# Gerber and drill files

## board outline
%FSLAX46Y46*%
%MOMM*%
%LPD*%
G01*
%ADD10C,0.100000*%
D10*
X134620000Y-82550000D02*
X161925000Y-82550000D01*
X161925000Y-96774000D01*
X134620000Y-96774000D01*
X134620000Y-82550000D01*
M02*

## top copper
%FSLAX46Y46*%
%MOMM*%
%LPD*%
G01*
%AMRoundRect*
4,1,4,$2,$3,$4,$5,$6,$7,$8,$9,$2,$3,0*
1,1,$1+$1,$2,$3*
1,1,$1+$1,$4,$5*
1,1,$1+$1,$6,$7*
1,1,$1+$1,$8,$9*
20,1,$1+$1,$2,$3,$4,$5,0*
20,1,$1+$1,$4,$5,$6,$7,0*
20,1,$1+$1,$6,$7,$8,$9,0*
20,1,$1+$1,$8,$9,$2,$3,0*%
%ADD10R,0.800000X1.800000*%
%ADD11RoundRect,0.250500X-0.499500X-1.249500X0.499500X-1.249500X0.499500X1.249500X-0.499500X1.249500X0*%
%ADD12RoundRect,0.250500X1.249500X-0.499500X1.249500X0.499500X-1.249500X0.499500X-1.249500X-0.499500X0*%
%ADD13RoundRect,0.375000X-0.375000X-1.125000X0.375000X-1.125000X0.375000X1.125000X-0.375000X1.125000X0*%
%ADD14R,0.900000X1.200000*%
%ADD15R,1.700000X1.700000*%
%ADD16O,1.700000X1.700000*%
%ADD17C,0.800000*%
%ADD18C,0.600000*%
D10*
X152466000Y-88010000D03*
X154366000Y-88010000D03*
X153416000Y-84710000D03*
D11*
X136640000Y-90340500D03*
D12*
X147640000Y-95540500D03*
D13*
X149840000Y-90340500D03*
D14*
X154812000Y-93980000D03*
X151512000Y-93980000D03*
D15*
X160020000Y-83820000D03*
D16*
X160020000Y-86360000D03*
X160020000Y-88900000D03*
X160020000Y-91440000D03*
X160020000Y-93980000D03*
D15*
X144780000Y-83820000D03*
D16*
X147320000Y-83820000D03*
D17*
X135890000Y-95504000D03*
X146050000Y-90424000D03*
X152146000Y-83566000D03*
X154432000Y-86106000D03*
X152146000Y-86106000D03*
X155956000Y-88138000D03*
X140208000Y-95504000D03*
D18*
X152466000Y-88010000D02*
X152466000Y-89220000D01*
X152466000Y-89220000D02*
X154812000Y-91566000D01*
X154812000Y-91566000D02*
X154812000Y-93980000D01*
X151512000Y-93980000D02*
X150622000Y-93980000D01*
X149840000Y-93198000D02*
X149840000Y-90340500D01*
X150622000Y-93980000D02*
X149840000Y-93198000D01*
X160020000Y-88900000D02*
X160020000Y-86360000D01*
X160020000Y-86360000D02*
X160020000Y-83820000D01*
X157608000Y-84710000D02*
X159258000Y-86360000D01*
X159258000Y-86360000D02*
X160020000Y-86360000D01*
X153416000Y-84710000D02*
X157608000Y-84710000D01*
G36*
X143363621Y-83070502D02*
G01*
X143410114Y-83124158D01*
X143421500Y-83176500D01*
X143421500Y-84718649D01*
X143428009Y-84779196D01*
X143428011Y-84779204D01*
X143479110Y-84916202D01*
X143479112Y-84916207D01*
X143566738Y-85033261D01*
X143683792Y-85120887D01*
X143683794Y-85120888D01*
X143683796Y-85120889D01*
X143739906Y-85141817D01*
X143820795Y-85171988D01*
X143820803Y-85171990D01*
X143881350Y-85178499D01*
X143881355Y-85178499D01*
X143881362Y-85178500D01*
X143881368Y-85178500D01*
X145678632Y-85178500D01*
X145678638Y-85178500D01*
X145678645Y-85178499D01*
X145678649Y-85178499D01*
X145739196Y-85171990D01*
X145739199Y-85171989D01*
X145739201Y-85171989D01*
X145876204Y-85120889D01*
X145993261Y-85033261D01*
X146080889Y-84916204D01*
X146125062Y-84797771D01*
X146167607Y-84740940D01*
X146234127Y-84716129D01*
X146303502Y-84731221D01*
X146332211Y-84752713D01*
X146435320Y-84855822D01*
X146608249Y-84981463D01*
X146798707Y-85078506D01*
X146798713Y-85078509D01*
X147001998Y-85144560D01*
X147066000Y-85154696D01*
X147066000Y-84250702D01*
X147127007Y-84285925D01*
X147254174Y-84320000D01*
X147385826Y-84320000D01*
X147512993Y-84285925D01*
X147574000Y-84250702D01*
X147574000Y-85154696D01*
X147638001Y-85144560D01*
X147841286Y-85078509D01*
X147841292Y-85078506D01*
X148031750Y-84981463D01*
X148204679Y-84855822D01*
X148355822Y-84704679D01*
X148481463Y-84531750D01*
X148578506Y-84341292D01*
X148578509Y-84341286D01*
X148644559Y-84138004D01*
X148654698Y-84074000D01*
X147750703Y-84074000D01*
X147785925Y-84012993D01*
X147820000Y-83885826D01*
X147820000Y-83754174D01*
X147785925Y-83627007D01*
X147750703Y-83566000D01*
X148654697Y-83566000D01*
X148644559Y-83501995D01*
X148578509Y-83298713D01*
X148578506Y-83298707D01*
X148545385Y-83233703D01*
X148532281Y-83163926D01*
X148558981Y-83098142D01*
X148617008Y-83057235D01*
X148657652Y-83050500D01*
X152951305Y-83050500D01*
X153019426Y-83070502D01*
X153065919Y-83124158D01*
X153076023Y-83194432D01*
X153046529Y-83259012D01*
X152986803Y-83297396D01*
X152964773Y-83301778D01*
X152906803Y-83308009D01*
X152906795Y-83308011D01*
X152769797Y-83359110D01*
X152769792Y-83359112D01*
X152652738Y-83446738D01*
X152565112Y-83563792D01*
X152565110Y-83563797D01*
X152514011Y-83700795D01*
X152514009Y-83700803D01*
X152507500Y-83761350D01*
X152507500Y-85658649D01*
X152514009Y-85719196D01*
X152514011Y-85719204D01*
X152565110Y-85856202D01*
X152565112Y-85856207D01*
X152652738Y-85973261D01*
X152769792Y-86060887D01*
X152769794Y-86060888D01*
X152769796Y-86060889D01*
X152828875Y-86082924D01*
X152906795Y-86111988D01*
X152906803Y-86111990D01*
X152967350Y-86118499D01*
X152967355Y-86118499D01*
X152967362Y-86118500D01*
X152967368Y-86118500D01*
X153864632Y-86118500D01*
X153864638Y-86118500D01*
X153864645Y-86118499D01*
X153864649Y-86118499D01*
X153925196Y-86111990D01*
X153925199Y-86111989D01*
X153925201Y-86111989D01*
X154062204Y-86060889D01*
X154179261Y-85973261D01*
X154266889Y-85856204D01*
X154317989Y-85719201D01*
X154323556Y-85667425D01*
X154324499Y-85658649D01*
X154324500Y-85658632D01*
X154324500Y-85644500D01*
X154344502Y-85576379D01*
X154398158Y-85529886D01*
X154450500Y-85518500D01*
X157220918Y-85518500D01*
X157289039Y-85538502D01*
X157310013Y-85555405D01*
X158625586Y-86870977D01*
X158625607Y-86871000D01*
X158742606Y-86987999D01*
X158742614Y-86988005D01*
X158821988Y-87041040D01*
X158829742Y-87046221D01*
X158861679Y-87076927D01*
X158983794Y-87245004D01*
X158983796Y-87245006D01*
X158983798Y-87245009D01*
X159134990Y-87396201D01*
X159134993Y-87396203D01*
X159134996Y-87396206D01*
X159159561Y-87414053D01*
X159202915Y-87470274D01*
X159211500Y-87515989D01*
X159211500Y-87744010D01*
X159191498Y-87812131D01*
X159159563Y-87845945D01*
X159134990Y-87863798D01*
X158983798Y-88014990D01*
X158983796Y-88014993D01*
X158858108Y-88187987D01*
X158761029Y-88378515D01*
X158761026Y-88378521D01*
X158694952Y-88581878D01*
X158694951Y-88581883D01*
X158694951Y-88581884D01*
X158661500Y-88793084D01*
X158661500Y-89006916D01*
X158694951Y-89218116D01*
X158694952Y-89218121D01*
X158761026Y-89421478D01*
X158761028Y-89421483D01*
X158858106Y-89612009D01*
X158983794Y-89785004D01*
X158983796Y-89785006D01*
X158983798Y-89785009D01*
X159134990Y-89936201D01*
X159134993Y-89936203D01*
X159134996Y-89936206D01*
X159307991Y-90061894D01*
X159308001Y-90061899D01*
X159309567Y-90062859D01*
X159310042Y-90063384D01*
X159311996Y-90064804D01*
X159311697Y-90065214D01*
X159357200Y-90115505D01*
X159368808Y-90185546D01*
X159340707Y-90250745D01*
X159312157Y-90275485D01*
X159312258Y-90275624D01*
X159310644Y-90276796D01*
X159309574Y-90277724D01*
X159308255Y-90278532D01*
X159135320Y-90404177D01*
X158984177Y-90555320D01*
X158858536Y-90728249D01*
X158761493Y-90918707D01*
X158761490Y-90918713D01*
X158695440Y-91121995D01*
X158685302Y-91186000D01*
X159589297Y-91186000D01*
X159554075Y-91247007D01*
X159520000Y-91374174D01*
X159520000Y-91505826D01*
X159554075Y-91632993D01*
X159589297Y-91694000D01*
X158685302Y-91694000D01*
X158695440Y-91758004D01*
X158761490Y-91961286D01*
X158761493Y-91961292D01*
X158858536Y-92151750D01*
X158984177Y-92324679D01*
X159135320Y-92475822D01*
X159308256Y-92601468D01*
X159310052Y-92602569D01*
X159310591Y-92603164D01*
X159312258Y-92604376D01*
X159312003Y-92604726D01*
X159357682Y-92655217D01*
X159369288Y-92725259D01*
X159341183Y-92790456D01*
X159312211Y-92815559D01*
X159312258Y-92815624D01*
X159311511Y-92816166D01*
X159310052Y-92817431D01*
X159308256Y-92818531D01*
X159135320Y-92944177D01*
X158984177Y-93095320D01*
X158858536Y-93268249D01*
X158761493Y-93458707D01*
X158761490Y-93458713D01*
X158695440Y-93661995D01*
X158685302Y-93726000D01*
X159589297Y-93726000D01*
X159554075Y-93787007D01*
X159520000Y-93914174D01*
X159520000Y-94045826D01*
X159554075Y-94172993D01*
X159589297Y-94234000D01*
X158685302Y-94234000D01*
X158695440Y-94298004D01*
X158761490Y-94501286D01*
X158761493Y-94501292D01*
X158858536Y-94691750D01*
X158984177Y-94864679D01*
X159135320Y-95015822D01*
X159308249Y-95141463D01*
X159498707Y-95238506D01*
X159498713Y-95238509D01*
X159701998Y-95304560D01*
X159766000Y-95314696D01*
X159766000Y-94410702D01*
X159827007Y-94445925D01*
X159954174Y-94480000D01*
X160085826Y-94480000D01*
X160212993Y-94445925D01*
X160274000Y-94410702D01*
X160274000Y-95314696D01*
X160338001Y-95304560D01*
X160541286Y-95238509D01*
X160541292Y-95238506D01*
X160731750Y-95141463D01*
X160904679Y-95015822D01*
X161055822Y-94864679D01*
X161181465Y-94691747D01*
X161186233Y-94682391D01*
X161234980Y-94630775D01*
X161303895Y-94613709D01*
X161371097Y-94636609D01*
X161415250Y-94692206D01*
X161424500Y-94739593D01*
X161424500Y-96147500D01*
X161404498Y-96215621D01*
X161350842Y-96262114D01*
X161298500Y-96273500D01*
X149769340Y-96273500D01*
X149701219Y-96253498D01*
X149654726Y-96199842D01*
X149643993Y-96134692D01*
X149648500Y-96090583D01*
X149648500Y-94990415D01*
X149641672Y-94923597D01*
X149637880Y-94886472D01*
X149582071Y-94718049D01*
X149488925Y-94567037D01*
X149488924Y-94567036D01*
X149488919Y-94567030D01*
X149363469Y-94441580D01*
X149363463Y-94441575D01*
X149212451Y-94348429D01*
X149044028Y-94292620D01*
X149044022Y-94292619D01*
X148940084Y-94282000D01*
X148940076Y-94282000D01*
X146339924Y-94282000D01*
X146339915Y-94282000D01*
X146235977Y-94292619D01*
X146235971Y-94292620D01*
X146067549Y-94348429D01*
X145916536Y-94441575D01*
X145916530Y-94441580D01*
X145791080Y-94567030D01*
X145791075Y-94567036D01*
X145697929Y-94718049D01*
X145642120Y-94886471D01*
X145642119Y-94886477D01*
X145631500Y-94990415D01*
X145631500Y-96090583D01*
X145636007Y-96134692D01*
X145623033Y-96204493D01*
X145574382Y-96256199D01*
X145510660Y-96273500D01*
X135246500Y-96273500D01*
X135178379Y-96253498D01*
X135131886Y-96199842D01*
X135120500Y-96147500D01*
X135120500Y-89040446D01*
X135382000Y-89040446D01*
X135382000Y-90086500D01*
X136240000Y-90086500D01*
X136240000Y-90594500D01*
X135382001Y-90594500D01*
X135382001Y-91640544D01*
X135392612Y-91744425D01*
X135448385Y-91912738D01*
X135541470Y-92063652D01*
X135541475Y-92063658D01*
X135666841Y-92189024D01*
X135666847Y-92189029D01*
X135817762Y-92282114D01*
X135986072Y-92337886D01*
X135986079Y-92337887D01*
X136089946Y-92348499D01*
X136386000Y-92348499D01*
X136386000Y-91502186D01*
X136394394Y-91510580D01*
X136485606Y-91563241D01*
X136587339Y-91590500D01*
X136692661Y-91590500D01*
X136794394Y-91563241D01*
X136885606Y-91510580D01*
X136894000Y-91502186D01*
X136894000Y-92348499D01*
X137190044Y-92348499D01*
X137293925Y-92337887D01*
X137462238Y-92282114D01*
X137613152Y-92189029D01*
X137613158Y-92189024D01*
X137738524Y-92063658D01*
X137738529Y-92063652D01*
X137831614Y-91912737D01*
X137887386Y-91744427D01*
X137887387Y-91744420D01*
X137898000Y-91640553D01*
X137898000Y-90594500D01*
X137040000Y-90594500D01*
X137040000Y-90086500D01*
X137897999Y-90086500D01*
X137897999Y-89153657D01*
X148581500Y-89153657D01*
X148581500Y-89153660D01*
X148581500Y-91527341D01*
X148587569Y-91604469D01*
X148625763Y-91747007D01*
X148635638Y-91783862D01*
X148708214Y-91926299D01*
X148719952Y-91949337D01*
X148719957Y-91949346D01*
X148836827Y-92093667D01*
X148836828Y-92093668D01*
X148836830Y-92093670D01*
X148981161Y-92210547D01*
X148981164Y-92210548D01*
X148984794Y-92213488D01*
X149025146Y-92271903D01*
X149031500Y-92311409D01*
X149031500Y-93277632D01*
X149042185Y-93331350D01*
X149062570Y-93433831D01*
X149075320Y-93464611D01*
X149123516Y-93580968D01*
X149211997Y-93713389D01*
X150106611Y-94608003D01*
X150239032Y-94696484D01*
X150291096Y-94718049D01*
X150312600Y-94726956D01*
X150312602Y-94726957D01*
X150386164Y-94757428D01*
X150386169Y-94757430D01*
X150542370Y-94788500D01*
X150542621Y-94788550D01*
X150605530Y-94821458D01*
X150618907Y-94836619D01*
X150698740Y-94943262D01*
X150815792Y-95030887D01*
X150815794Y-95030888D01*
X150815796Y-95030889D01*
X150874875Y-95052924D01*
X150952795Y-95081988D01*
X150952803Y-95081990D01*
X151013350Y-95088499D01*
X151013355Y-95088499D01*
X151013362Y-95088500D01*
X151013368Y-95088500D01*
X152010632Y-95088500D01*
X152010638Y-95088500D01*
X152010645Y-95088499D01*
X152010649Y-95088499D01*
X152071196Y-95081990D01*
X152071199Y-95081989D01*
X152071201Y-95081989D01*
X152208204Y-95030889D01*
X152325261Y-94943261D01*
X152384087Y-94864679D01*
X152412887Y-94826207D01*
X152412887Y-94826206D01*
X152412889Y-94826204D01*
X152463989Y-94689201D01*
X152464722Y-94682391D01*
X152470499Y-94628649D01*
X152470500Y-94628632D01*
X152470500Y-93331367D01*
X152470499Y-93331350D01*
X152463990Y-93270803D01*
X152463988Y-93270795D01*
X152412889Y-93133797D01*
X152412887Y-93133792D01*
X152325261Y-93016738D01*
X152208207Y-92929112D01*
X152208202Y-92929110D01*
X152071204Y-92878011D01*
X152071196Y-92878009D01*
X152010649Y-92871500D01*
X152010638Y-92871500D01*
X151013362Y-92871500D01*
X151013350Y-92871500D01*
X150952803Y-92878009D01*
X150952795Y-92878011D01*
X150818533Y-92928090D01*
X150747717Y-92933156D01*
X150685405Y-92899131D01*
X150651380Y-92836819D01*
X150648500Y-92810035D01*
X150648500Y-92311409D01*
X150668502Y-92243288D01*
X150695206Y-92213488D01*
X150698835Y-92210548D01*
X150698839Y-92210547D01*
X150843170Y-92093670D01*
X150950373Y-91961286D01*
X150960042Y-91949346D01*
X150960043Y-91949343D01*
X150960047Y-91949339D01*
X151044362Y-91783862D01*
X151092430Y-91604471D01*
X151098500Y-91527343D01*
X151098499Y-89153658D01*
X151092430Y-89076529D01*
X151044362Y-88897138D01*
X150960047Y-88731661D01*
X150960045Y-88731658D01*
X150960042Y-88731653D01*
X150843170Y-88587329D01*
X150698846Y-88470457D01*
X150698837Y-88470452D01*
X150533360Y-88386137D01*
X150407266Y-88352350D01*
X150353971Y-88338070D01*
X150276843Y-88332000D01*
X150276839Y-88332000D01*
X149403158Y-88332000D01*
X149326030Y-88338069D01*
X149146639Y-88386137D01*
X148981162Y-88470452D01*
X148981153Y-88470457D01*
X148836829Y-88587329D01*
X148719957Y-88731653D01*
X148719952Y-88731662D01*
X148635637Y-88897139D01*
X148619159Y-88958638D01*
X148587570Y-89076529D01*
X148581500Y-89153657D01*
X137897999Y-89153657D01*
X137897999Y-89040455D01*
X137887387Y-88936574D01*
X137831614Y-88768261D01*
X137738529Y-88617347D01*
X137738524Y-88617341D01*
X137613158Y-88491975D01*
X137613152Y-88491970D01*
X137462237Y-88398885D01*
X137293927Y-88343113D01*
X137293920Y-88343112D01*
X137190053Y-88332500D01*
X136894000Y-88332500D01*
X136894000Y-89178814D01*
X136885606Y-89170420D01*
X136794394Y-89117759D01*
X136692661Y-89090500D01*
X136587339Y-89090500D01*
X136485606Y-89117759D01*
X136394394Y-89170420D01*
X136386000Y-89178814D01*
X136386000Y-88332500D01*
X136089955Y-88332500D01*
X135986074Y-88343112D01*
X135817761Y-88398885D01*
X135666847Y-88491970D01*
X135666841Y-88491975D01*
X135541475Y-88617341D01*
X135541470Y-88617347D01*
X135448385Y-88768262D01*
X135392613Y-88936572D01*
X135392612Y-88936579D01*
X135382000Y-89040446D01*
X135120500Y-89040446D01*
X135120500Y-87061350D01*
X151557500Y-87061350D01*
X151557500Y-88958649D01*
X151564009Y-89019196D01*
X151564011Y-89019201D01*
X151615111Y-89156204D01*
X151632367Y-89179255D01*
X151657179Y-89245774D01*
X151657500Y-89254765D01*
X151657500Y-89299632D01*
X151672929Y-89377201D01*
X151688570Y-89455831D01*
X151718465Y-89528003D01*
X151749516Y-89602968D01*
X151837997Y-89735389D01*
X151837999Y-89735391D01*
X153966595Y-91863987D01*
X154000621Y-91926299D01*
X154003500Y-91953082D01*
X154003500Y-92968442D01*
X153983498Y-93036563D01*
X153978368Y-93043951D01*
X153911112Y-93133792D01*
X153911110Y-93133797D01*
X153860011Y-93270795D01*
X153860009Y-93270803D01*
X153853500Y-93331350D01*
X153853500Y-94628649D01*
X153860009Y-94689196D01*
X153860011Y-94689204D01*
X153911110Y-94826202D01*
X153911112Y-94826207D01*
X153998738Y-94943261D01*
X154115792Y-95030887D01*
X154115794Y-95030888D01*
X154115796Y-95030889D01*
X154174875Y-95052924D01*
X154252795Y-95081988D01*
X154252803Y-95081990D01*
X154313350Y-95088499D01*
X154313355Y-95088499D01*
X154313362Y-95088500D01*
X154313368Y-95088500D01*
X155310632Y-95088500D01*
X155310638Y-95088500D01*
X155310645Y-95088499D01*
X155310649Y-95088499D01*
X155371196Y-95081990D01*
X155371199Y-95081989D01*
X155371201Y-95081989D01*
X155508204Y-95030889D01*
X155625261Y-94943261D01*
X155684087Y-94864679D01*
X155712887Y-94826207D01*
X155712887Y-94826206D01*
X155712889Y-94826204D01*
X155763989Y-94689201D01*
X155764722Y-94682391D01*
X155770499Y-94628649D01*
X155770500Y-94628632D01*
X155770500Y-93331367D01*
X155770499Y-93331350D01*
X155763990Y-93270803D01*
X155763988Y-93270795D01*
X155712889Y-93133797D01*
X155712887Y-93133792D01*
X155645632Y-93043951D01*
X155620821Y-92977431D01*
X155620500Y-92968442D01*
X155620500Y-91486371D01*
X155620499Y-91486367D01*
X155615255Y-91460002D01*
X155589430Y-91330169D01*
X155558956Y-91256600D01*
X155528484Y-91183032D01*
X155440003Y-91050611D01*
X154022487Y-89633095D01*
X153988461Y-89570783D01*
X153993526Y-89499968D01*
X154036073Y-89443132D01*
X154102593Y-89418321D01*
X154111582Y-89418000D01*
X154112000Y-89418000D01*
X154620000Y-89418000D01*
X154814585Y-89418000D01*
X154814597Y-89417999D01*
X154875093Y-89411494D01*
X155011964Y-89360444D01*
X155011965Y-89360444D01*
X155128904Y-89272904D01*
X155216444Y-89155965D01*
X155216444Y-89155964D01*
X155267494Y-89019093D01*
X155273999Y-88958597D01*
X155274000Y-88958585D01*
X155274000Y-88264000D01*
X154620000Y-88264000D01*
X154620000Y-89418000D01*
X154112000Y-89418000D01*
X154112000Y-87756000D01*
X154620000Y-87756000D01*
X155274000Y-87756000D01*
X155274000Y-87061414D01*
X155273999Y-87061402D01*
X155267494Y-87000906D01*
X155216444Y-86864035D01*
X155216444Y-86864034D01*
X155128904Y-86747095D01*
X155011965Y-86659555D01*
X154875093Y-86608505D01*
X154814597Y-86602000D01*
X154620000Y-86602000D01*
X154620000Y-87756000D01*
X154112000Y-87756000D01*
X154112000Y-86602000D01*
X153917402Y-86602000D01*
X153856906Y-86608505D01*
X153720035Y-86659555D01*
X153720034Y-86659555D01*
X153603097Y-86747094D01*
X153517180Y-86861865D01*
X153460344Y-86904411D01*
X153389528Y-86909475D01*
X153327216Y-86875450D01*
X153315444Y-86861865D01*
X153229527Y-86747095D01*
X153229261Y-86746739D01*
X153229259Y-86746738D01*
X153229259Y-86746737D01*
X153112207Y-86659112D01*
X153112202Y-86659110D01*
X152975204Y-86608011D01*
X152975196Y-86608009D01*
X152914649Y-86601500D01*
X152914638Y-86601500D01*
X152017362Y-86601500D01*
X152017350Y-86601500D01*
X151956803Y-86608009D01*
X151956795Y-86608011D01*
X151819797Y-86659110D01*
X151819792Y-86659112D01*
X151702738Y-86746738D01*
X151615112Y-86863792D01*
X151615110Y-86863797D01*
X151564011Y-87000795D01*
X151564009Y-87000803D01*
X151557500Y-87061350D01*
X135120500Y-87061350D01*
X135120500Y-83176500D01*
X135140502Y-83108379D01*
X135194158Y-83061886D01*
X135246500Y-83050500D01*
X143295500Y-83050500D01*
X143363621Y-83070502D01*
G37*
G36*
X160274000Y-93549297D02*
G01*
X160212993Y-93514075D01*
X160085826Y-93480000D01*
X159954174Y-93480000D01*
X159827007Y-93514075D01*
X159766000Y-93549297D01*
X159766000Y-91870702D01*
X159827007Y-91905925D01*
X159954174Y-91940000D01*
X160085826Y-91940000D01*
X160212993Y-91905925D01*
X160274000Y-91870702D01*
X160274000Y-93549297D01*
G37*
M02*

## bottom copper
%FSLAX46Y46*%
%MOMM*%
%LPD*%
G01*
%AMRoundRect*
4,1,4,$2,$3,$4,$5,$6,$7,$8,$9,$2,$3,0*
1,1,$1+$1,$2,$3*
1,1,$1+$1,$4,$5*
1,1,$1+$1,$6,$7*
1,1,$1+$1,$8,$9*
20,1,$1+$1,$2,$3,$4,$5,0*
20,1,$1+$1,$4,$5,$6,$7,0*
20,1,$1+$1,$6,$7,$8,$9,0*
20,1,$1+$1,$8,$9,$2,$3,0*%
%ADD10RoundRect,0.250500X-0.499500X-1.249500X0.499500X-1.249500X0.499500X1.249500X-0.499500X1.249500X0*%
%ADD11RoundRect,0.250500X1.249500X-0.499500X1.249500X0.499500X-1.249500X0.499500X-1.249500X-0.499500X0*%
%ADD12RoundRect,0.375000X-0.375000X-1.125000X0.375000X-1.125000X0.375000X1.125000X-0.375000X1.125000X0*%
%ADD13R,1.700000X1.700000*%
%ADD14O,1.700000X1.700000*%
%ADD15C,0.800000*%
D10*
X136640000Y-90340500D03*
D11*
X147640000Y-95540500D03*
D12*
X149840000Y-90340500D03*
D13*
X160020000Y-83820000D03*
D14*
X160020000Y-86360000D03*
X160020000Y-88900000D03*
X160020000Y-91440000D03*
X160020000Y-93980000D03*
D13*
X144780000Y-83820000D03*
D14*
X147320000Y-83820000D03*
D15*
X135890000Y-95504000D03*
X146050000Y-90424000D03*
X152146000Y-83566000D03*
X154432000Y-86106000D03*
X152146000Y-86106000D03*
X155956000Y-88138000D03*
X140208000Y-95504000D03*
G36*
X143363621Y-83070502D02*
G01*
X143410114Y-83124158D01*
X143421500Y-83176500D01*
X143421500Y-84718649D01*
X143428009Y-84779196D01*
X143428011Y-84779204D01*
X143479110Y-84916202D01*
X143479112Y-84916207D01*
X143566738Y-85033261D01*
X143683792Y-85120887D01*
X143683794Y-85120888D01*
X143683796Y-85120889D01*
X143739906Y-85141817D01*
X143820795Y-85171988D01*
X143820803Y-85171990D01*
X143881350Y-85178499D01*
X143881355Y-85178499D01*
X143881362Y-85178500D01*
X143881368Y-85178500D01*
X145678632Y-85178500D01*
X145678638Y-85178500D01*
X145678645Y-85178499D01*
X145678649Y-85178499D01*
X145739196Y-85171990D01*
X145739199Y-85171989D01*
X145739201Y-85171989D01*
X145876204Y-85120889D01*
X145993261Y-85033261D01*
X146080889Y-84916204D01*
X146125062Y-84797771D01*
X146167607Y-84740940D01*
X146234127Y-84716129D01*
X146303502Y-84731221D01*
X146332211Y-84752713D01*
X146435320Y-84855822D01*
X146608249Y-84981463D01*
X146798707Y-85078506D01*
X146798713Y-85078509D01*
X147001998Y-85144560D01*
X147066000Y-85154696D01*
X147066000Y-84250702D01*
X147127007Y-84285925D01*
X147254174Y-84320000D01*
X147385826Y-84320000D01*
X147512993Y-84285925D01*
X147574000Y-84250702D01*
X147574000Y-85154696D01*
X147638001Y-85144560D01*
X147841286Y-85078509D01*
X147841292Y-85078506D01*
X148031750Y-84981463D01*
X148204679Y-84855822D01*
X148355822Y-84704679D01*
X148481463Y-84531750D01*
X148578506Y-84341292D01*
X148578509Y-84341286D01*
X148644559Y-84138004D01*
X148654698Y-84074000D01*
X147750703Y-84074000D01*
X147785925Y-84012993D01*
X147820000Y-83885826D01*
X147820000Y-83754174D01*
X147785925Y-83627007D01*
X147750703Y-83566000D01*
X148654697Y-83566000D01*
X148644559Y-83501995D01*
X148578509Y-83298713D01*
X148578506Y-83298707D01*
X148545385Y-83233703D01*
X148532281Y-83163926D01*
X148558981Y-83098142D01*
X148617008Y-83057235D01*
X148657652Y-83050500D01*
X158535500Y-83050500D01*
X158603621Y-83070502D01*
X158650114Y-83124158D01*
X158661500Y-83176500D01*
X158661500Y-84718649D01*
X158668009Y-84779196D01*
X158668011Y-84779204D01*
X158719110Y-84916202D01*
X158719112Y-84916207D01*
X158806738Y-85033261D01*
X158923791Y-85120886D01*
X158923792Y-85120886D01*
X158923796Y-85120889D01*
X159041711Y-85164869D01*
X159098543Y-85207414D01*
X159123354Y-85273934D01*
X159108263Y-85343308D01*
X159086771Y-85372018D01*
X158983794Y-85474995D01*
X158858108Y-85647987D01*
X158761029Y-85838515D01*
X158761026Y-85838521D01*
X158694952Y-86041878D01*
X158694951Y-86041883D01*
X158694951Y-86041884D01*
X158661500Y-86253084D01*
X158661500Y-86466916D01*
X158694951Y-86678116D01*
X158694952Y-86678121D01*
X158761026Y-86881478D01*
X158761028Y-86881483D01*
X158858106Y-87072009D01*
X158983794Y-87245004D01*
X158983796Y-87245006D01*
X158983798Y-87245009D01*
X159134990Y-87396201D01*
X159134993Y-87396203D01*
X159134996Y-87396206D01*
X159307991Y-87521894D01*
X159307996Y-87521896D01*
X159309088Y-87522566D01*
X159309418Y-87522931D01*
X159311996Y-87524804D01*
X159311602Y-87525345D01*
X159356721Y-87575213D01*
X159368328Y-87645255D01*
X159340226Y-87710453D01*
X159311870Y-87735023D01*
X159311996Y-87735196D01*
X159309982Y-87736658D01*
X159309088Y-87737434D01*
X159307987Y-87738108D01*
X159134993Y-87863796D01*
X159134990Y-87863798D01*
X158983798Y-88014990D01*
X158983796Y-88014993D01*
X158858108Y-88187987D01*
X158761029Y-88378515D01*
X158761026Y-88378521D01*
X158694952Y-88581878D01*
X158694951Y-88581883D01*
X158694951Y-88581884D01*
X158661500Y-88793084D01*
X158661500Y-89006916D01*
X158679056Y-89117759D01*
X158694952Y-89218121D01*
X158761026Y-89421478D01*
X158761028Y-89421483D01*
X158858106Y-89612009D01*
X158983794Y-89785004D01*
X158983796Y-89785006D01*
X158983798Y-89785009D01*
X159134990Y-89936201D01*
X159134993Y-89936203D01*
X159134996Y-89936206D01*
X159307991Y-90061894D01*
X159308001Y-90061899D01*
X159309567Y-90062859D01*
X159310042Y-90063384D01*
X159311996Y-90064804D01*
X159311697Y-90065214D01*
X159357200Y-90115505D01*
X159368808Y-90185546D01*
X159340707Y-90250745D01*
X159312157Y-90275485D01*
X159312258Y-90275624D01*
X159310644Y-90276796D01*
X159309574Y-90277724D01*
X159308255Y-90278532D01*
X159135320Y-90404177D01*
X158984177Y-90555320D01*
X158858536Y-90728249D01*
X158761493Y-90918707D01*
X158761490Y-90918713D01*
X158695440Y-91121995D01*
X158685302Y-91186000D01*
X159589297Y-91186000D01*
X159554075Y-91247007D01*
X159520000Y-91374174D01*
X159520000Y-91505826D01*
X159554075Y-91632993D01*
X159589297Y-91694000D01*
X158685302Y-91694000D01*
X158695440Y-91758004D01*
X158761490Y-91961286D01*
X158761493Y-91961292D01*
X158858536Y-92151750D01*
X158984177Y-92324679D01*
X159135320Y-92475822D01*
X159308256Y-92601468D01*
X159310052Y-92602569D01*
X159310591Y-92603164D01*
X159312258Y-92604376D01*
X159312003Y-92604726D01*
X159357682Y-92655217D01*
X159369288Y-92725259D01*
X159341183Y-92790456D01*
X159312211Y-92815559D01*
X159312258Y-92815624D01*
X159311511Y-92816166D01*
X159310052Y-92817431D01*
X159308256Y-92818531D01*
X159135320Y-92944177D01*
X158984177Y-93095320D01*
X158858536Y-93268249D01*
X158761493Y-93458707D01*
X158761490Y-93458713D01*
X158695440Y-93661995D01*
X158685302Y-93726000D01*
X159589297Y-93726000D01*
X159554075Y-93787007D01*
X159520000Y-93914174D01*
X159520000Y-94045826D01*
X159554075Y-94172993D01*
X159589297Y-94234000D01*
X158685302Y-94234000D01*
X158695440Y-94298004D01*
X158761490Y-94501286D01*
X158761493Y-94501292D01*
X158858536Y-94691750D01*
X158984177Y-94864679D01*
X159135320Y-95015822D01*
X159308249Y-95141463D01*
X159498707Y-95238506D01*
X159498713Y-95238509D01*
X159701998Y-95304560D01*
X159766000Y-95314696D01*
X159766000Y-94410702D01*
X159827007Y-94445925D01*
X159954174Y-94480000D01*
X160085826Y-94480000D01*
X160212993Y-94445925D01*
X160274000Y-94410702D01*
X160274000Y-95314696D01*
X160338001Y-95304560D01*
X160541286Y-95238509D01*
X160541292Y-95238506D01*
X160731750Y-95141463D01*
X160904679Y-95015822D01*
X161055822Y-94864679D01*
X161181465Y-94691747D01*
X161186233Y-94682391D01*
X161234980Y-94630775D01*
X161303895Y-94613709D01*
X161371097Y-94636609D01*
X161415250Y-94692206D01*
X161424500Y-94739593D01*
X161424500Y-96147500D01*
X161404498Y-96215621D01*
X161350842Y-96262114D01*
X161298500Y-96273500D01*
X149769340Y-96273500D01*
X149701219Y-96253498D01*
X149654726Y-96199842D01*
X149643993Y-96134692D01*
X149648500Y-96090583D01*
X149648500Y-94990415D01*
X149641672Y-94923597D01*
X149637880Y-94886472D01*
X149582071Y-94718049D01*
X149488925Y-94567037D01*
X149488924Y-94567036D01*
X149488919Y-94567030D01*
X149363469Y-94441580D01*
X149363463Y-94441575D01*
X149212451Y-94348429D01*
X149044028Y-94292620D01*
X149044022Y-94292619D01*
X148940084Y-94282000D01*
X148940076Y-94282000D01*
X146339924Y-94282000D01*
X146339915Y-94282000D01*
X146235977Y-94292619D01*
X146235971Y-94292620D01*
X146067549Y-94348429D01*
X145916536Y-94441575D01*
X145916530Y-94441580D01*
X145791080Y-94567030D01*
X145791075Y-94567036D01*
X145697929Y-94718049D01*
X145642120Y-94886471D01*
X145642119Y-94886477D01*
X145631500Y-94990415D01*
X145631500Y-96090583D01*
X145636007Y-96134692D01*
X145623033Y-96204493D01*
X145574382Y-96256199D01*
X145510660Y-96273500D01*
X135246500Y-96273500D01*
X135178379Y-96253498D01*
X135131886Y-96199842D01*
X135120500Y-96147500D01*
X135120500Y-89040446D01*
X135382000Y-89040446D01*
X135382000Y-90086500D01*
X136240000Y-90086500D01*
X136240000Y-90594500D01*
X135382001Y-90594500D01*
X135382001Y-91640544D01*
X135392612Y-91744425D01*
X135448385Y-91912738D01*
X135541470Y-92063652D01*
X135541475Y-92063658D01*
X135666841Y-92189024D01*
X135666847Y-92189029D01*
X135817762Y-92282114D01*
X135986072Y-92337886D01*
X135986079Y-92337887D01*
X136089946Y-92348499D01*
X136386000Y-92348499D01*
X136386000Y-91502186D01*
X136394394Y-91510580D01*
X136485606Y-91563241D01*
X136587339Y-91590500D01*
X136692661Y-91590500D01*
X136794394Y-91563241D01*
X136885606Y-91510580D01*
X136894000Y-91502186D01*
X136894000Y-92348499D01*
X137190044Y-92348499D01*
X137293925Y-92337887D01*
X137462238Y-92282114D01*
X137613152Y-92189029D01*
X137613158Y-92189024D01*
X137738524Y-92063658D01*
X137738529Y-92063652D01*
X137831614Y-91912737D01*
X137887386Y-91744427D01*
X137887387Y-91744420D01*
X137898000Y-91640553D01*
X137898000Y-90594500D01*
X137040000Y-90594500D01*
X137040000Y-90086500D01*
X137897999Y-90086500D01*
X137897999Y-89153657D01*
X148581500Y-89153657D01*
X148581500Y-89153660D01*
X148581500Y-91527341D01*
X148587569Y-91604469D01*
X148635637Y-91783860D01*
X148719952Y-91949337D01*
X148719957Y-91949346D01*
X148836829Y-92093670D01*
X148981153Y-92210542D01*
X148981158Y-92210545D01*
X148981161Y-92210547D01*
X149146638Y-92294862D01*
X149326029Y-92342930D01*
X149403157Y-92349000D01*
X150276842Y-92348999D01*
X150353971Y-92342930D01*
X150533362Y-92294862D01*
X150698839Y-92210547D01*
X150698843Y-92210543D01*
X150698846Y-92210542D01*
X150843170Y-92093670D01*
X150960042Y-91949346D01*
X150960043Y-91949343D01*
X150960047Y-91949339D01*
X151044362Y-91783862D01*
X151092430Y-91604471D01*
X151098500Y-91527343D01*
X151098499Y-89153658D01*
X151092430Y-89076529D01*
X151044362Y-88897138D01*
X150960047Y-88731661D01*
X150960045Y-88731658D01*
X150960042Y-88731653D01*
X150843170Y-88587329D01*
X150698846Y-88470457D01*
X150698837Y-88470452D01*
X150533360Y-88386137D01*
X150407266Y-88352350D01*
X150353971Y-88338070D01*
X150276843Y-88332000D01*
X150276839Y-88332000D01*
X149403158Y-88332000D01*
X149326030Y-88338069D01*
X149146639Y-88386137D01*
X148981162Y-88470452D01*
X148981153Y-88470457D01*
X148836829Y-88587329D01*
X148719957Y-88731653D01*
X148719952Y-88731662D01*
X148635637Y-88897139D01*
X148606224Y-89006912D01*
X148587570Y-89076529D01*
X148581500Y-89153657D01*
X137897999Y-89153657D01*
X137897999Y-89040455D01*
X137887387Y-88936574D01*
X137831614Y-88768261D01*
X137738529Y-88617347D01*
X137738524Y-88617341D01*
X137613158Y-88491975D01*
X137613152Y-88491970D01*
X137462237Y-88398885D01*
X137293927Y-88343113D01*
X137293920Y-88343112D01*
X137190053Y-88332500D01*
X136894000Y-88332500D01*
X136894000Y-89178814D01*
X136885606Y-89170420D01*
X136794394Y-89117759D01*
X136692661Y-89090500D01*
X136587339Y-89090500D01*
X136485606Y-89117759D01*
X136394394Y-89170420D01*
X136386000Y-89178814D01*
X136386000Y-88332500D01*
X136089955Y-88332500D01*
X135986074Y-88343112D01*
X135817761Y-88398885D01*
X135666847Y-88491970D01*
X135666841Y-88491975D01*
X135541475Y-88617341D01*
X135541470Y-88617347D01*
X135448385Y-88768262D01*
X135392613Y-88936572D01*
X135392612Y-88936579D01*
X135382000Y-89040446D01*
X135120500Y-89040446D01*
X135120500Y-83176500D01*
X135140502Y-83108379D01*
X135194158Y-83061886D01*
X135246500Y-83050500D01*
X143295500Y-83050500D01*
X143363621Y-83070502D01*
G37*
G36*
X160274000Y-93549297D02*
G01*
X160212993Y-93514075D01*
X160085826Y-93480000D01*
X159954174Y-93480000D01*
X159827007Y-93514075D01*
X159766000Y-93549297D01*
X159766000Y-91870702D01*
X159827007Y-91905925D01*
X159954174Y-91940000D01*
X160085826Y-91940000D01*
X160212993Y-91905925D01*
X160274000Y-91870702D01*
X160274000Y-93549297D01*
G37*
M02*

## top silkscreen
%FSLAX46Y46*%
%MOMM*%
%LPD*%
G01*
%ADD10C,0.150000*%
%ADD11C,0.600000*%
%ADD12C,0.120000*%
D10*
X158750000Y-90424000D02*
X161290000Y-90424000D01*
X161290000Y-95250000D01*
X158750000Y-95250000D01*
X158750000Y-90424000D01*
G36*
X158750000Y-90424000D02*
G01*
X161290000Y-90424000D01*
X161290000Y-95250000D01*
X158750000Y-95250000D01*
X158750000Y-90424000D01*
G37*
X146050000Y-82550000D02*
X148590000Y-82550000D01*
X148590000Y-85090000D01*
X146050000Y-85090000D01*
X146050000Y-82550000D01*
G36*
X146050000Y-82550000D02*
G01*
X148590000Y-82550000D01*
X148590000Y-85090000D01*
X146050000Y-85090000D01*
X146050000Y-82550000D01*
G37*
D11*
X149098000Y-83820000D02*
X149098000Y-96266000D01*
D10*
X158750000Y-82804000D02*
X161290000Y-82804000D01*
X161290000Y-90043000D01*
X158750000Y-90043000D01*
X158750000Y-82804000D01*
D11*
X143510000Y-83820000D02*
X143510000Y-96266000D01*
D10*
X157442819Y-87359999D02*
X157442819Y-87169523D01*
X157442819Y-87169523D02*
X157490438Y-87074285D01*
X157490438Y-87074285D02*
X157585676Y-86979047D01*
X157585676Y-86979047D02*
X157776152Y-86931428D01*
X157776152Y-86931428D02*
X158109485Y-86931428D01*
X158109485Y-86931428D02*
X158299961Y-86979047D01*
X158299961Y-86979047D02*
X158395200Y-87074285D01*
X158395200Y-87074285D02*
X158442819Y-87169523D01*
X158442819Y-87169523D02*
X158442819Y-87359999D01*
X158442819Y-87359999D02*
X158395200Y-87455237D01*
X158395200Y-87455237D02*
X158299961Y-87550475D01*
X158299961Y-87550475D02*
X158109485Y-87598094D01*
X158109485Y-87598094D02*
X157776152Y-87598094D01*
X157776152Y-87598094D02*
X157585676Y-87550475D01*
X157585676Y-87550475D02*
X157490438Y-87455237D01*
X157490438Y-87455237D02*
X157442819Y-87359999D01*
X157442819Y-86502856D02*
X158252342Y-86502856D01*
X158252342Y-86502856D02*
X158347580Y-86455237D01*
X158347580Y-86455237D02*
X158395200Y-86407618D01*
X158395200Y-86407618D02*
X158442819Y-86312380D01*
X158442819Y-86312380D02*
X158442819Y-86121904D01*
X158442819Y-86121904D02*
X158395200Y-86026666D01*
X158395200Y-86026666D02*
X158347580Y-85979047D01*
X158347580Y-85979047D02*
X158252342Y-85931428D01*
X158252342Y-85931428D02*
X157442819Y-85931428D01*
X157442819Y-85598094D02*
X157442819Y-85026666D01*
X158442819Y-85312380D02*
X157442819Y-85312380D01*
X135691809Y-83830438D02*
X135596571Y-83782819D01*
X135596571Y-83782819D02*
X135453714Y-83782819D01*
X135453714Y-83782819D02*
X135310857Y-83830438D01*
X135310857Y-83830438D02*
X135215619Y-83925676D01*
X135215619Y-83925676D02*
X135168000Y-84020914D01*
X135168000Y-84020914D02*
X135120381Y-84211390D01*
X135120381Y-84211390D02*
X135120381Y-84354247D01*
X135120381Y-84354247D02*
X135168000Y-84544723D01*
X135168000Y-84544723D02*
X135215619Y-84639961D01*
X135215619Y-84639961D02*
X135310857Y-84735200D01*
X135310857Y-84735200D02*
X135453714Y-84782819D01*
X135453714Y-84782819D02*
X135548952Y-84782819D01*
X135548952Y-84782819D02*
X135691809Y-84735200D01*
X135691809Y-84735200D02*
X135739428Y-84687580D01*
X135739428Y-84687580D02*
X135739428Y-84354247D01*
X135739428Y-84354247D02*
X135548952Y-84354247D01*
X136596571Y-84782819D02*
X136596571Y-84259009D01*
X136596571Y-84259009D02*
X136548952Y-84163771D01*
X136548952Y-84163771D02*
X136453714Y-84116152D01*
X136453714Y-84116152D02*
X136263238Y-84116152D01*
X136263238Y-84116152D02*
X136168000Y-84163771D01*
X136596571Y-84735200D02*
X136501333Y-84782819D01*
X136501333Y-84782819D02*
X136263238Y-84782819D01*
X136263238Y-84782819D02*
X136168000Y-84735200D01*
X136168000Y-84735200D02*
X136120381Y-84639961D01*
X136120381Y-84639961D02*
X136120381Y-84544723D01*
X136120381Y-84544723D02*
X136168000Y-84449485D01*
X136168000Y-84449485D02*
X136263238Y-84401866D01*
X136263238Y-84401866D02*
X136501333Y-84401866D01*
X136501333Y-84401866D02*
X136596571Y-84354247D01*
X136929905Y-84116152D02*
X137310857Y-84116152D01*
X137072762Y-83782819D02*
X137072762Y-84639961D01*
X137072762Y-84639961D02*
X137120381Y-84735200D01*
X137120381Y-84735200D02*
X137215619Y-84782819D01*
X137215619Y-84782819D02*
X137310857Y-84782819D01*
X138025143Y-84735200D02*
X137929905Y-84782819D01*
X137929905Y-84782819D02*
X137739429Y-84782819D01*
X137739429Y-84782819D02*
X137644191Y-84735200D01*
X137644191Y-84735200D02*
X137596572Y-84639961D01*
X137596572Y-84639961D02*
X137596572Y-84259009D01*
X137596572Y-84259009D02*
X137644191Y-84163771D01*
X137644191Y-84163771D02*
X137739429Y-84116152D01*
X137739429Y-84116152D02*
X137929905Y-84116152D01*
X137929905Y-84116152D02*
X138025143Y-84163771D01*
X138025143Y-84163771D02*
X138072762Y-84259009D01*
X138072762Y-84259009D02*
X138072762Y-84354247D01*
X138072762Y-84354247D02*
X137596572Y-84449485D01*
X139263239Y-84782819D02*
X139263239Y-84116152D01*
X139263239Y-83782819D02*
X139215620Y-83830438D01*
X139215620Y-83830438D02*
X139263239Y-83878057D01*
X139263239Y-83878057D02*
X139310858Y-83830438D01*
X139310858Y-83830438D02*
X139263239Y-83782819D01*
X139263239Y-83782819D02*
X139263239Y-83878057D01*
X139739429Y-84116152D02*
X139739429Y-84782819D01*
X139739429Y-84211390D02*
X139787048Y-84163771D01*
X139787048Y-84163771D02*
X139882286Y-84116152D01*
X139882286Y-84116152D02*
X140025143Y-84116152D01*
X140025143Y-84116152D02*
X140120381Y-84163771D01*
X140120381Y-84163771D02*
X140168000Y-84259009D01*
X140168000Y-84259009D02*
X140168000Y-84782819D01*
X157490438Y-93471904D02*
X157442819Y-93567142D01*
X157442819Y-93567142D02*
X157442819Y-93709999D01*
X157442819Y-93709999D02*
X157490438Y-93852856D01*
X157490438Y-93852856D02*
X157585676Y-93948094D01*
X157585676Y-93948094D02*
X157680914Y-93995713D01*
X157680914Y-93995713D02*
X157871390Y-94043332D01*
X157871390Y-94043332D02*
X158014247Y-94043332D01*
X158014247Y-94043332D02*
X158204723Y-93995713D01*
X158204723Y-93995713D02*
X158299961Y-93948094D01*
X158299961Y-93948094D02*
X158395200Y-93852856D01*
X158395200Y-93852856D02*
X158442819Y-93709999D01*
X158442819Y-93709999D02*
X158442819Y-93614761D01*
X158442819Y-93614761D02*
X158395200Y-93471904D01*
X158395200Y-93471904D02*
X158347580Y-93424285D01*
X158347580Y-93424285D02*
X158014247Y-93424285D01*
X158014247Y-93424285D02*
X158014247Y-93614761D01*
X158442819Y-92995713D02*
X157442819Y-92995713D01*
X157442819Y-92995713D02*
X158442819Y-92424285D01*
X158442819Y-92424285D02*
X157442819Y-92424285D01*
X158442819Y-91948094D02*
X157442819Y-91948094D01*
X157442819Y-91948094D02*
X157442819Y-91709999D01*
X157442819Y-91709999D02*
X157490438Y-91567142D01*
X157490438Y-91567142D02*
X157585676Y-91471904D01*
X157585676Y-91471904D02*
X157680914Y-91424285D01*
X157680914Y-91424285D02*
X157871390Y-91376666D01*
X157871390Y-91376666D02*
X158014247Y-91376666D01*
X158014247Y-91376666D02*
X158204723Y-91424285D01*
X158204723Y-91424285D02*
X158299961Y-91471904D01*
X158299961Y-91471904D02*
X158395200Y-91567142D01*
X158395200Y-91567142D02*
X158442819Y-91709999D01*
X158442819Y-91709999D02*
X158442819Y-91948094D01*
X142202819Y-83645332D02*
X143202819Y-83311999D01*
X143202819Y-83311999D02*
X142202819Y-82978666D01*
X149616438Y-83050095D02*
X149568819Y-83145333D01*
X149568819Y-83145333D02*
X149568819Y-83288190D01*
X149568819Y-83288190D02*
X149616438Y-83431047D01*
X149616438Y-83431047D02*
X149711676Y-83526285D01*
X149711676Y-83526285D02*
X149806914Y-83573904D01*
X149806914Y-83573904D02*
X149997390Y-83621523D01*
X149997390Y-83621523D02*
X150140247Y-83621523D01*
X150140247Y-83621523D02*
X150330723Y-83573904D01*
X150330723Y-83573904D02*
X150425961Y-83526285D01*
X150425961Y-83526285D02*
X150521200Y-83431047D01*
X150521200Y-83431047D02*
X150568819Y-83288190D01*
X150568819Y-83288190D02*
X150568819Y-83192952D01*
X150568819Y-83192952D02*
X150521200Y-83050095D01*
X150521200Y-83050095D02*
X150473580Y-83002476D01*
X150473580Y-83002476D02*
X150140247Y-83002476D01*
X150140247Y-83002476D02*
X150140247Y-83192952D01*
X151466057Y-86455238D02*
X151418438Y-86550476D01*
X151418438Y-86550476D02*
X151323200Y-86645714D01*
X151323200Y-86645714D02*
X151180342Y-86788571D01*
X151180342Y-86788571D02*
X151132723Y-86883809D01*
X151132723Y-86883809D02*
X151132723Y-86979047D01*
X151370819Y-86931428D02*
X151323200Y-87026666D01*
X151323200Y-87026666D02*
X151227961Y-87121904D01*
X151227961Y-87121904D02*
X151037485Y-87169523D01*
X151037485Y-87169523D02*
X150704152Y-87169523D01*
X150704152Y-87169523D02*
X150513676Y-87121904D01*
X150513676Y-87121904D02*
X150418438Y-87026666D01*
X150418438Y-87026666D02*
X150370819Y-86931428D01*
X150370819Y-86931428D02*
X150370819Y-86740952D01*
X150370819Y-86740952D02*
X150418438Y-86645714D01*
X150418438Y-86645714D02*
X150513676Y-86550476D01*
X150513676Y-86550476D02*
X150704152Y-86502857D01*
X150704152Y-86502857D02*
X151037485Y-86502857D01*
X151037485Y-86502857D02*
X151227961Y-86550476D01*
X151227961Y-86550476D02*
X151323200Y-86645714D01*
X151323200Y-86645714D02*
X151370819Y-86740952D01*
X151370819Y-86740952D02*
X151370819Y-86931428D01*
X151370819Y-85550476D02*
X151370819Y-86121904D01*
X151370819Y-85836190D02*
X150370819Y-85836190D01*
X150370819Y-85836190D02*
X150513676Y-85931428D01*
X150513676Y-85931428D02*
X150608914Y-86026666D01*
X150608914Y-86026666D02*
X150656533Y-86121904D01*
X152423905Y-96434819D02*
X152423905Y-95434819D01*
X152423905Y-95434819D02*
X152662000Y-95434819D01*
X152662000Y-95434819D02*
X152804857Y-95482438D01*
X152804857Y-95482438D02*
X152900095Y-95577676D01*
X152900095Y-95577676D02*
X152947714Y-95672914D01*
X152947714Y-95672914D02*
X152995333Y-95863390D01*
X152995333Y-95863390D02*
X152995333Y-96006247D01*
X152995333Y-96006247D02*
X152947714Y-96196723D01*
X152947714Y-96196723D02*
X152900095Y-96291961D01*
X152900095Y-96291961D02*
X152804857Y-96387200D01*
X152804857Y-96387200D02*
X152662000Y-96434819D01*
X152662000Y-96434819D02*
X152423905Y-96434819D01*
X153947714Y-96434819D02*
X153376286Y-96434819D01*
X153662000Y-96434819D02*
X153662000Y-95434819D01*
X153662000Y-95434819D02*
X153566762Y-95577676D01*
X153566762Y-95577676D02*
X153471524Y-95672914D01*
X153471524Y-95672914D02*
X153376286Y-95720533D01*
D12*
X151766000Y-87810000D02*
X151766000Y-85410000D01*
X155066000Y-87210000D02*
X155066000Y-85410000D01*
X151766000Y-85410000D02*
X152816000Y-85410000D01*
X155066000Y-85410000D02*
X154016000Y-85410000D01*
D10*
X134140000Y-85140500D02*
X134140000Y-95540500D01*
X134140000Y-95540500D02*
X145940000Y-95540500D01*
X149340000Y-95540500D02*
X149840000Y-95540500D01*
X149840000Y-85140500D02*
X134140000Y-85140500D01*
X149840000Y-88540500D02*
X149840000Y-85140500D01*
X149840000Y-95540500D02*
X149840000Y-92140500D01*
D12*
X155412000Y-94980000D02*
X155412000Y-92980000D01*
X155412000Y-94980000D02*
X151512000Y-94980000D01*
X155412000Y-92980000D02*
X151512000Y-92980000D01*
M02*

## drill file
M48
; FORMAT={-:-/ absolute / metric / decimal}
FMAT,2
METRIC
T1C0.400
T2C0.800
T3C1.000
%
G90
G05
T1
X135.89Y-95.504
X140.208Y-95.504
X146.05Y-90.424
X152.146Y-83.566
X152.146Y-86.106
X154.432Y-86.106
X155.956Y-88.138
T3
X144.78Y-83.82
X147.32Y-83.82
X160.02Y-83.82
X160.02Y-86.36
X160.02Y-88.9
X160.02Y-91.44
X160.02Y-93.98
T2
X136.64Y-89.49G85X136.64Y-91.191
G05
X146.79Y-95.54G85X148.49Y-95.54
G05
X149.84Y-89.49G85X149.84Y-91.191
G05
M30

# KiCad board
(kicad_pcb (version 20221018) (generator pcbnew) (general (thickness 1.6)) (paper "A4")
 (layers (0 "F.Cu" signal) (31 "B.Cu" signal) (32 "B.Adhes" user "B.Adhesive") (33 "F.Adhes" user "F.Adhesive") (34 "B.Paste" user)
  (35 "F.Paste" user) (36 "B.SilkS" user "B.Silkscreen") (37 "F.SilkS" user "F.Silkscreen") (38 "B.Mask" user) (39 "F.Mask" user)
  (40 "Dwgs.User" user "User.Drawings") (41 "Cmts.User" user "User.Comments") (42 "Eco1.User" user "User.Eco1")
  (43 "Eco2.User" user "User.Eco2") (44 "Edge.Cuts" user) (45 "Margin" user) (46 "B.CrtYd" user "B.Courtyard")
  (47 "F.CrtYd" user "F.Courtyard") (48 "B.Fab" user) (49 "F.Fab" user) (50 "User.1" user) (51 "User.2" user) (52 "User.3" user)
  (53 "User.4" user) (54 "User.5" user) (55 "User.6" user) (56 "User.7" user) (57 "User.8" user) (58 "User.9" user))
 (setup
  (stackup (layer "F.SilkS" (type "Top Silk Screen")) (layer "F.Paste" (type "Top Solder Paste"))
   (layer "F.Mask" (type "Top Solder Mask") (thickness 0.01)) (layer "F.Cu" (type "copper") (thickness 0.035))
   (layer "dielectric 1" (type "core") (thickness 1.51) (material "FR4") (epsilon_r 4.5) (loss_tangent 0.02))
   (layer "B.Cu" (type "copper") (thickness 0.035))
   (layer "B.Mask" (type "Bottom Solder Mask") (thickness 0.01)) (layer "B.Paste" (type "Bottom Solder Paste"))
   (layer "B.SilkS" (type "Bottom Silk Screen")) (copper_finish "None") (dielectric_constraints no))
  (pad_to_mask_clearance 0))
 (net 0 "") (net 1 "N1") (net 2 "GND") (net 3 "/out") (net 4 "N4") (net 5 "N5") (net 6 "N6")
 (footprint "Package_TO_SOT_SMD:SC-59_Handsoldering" (layer "F.Cu") (at 153.416 86.36 90)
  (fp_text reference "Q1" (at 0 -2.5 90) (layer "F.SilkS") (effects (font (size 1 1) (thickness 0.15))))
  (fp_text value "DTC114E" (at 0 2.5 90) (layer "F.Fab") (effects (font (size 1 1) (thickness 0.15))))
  (fp_line (start -1.45 -1.65) (end 0.95 -1.65) (stroke (width 0.12) (type solid)) (layer "F.SilkS"))
  (fp_line (start -0.85 1.65) (end 0.95 1.65) (stroke (width 0.12) (type solid)) (layer "F.SilkS"))
  (fp_line (start 0.95 -1.65) (end 0.95 -0.6) (stroke (width 0.12) (type solid)) (layer "F.SilkS"))
  (fp_line (start 0.95 1.65) (end 0.95 0.6) (stroke (width 0.12) (type solid)) (layer "F.SilkS"))
  (pad "1" smd rect (at -1.65 -0.95 90) (size 1.8 0.8) (layers "F.Cu" "F.Paste" "F.Mask") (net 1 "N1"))
  (pad "2" smd rect (at -1.65 0.95 90) (size 1.8 0.8) (layers "F.Cu" "F.Paste" "F.Mask") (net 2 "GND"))
  (pad "3" smd rect (at 1.65 0 90) (size 1.8 0.8) (layers "F.Cu" "F.Paste" "F.Mask") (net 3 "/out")))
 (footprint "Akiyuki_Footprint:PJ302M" (layer "F.Cu") (at 134.14 90.3405)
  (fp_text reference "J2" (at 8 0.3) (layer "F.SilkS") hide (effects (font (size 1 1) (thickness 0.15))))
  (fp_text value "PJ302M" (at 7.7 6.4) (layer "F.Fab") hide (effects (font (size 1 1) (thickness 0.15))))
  (fp_line (start 0 -5.2) (end 0 5.2) (stroke (width 0.15) (type solid)) (layer "F.SilkS"))
  (fp_line (start 0 5.2) (end 11.8 5.2) (stroke (width 0.15) (type solid)) (layer "F.SilkS"))
  (fp_line (start 15.2 5.2) (end 15.7 5.2) (stroke (width 0.15) (type solid)) (layer "F.SilkS"))
  (fp_line (start 15.7 -5.2) (end 0 -5.2) (stroke (width 0.15) (type solid)) (layer "F.SilkS"))
  (fp_line (start 15.7 -1.8) (end 15.7 -5.2) (stroke (width 0.15) (type solid)) (layer "F.SilkS"))
  (fp_line (start 15.7 5.2) (end 15.7 1.8) (stroke (width 0.15) (type solid)) (layer "F.SilkS"))
  (pad "1" thru_hole roundrect (at 2.5 0) (size 1.5 3) (drill oval 0.8 2.5) (layers "*.Cu" "*.Mask") (roundrect_rratio 0.167) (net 2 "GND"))
  (pad "2" thru_hole roundrect (at 13.5 5.2 90) (size 1.5 3) (drill oval 0.8 2.5) (layers "*.Cu" "*.Mask") (roundrect_rratio 0.167)
   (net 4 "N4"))
  (pad "3" thru_hole roundrect (at 15.7 0) (size 1.5 3) (drill oval 0.8 2.5) (layers "*.Cu" "*.Mask") (roundrect_rratio 0.25) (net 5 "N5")))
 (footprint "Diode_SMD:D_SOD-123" (layer "F.Cu") (at 153.162 93.98 180)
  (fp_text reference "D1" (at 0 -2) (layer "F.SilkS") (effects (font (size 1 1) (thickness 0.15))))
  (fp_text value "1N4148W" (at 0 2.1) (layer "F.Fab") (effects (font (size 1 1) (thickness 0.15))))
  (fp_line (start -2.25 -1) (end -2.25 1) (stroke (width 0.12) (type solid)) (layer "F.SilkS"))
  (fp_line (start -2.25 -1) (end 1.65 -1) (stroke (width 0.12) (type solid)) (layer "F.SilkS"))
  (fp_line (start -2.25 1) (end 1.65 1) (stroke (width 0.12) (type solid)) (layer "F.SilkS"))
  (pad "1" smd rect (at -1.65 0 180) (size 0.9 1.2) (layers "F.Cu" "F.Paste" "F.Mask") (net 1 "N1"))
  (pad "2" smd rect (at 1.65 0 180) (size 0.9 1.2) (layers "F.Cu" "F.Paste" "F.Mask") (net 5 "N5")))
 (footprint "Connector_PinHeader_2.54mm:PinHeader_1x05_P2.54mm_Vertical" (layer "B.Cu") (at 160.02 83.82 180)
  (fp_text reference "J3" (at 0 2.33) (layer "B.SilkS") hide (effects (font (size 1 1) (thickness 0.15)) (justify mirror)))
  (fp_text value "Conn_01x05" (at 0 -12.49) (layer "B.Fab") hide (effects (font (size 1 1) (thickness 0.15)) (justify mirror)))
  (pad "1" thru_hole rect (at 0 0 180) (size 1.7 1.7) (drill 1) (layers "*.Cu" "*.Mask") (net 3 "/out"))
  (pad "2" thru_hole oval (at 0 -2.54 180) (size 1.7 1.7) (drill 1) (layers "*.Cu" "*.Mask") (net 3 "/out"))
  (pad "3" thru_hole oval (at 0 -5.08 180) (size 1.7 1.7) (drill 1) (layers "*.Cu" "*.Mask") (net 3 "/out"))
  (pad "4" thru_hole oval (at 0 -7.62 180) (size 1.7 1.7) (drill 1) (layers "*.Cu" "*.Mask") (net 2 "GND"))
  (pad "5" thru_hole oval (at 0 -10.16 180) (size 1.7 1.7) (drill 1) (layers "*.Cu" "*.Mask") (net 2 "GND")))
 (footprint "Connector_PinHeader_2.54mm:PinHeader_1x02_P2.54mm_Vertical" (layer "B.Cu") (at 144.78 83.82 -90)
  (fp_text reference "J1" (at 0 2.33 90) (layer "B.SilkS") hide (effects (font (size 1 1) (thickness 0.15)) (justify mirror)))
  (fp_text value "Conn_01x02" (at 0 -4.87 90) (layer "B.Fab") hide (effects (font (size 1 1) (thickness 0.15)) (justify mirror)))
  (pad "1" thru_hole rect (at 0 0 270) (size 1.7 1.7) (drill 1) (layers "*.Cu" "*.Mask") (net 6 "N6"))
  (pad "2" thru_hole oval (at 0 -2.54 270) (size 1.7 1.7) (drill 1) (layers "*.Cu" "*.Mask") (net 2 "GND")))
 (gr_rect (start 158.75 90.424) (end 161.29 95.25) (stroke (width 0.15) (type solid)) (fill solid) (layer "F.SilkS"))
 (gr_rect (start 146.05 82.55) (end 148.59 85.09) (stroke (width 0.15) (type solid)) (fill solid) (layer "F.SilkS"))
 (gr_line (start 149.098 83.82) (end 149.098 96.266) (stroke (width 0.6) (type solid)) (layer "F.SilkS"))
 (gr_rect (start 158.75 82.804) (end 161.29 90.043) (stroke (width 0.15) (type solid)) (fill none) (layer "F.SilkS"))
 (gr_line (start 143.51 83.82) (end 143.51 96.266) (stroke (width 0.6) (type solid)) (layer "F.SilkS"))
 (gr_rect (start 134.62 82.55) (end 161.925 96.774) (stroke (width 0.1) (type solid)) (fill none) (layer "Edge.Cuts"))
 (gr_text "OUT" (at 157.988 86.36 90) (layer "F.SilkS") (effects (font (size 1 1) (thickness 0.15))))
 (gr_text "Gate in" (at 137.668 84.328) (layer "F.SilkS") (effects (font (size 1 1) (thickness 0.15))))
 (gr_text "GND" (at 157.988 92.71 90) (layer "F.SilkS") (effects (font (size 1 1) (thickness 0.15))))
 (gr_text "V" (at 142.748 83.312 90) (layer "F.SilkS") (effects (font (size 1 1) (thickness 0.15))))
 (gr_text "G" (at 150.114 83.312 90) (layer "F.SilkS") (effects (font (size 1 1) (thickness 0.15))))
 (segment (start 152.466 88.01) (end 152.466 89.22) (width 0.6) (layer "F.Cu") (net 1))
 (segment (start 152.466 89.22) (end 154.812 91.566) (width 0.6) (layer "F.Cu") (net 1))
 (segment (start 154.812 91.566) (end 154.812 93.98) (width 0.6) (layer "F.Cu") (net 1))
 (segment (start 151.512 93.98) (end 150.622 93.98) (width 0.6) (layer "F.Cu") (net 5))
 (segment (start 149.84 93.198) (end 149.84 90.3405) (width 0.6) (layer "F.Cu") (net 5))
 (segment (start 150.622 93.98) (end 149.84 93.198) (width 0.6) (layer "F.Cu") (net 5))
 (via (at 135.89 95.504) (size 0.8) (drill 0.4) (layers "F.Cu" "B.Cu") (free) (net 2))
 (via (at 146.05 90.424) (size 0.8) (drill 0.4) (layers "F.Cu" "B.Cu") (free) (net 2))
 (via (at 152.146 83.566) (size 0.8) (drill 0.4) (layers "F.Cu" "B.Cu") (free) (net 2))
 (via (at 154.432 86.106) (size 0.8) (drill 0.4) (layers "F.Cu" "B.Cu") (free) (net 2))
 (via (at 152.146 86.106) (size 0.8) (drill 0.4) (layers "F.Cu" "B.Cu") (free) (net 2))
 (via (at 155.956 88.138) (size 0.8) (drill 0.4) (layers "F.Cu" "B.Cu") (free) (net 2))
 (via (at 140.208 95.504) (size 0.8) (drill 0.4) (layers "F.Cu" "B.Cu") (free) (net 2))
 (segment (start 160.02 88.9) (end 160.02 86.36) (width 0.6) (layer "F.Cu") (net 3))
 (segment (start 160.02 86.36) (end 160.02 83.82) (width 0.6) (layer "F.Cu") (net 3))
 (segment (start 157.608 84.71) (end 159.258 86.36) (width 0.6) (layer "F.Cu") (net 3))
 (segment (start 159.258 86.36) (end 160.02 86.36) (width 0.6) (layer "F.Cu") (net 3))
 (segment (start 153.416 84.71) (end 157.608 84.71) (width 0.6) (layer "F.Cu") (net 3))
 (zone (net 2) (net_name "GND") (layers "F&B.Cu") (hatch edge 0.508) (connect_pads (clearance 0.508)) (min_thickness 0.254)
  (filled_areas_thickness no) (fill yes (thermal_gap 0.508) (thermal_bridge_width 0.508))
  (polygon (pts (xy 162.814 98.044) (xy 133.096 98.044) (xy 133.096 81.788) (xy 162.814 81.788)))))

